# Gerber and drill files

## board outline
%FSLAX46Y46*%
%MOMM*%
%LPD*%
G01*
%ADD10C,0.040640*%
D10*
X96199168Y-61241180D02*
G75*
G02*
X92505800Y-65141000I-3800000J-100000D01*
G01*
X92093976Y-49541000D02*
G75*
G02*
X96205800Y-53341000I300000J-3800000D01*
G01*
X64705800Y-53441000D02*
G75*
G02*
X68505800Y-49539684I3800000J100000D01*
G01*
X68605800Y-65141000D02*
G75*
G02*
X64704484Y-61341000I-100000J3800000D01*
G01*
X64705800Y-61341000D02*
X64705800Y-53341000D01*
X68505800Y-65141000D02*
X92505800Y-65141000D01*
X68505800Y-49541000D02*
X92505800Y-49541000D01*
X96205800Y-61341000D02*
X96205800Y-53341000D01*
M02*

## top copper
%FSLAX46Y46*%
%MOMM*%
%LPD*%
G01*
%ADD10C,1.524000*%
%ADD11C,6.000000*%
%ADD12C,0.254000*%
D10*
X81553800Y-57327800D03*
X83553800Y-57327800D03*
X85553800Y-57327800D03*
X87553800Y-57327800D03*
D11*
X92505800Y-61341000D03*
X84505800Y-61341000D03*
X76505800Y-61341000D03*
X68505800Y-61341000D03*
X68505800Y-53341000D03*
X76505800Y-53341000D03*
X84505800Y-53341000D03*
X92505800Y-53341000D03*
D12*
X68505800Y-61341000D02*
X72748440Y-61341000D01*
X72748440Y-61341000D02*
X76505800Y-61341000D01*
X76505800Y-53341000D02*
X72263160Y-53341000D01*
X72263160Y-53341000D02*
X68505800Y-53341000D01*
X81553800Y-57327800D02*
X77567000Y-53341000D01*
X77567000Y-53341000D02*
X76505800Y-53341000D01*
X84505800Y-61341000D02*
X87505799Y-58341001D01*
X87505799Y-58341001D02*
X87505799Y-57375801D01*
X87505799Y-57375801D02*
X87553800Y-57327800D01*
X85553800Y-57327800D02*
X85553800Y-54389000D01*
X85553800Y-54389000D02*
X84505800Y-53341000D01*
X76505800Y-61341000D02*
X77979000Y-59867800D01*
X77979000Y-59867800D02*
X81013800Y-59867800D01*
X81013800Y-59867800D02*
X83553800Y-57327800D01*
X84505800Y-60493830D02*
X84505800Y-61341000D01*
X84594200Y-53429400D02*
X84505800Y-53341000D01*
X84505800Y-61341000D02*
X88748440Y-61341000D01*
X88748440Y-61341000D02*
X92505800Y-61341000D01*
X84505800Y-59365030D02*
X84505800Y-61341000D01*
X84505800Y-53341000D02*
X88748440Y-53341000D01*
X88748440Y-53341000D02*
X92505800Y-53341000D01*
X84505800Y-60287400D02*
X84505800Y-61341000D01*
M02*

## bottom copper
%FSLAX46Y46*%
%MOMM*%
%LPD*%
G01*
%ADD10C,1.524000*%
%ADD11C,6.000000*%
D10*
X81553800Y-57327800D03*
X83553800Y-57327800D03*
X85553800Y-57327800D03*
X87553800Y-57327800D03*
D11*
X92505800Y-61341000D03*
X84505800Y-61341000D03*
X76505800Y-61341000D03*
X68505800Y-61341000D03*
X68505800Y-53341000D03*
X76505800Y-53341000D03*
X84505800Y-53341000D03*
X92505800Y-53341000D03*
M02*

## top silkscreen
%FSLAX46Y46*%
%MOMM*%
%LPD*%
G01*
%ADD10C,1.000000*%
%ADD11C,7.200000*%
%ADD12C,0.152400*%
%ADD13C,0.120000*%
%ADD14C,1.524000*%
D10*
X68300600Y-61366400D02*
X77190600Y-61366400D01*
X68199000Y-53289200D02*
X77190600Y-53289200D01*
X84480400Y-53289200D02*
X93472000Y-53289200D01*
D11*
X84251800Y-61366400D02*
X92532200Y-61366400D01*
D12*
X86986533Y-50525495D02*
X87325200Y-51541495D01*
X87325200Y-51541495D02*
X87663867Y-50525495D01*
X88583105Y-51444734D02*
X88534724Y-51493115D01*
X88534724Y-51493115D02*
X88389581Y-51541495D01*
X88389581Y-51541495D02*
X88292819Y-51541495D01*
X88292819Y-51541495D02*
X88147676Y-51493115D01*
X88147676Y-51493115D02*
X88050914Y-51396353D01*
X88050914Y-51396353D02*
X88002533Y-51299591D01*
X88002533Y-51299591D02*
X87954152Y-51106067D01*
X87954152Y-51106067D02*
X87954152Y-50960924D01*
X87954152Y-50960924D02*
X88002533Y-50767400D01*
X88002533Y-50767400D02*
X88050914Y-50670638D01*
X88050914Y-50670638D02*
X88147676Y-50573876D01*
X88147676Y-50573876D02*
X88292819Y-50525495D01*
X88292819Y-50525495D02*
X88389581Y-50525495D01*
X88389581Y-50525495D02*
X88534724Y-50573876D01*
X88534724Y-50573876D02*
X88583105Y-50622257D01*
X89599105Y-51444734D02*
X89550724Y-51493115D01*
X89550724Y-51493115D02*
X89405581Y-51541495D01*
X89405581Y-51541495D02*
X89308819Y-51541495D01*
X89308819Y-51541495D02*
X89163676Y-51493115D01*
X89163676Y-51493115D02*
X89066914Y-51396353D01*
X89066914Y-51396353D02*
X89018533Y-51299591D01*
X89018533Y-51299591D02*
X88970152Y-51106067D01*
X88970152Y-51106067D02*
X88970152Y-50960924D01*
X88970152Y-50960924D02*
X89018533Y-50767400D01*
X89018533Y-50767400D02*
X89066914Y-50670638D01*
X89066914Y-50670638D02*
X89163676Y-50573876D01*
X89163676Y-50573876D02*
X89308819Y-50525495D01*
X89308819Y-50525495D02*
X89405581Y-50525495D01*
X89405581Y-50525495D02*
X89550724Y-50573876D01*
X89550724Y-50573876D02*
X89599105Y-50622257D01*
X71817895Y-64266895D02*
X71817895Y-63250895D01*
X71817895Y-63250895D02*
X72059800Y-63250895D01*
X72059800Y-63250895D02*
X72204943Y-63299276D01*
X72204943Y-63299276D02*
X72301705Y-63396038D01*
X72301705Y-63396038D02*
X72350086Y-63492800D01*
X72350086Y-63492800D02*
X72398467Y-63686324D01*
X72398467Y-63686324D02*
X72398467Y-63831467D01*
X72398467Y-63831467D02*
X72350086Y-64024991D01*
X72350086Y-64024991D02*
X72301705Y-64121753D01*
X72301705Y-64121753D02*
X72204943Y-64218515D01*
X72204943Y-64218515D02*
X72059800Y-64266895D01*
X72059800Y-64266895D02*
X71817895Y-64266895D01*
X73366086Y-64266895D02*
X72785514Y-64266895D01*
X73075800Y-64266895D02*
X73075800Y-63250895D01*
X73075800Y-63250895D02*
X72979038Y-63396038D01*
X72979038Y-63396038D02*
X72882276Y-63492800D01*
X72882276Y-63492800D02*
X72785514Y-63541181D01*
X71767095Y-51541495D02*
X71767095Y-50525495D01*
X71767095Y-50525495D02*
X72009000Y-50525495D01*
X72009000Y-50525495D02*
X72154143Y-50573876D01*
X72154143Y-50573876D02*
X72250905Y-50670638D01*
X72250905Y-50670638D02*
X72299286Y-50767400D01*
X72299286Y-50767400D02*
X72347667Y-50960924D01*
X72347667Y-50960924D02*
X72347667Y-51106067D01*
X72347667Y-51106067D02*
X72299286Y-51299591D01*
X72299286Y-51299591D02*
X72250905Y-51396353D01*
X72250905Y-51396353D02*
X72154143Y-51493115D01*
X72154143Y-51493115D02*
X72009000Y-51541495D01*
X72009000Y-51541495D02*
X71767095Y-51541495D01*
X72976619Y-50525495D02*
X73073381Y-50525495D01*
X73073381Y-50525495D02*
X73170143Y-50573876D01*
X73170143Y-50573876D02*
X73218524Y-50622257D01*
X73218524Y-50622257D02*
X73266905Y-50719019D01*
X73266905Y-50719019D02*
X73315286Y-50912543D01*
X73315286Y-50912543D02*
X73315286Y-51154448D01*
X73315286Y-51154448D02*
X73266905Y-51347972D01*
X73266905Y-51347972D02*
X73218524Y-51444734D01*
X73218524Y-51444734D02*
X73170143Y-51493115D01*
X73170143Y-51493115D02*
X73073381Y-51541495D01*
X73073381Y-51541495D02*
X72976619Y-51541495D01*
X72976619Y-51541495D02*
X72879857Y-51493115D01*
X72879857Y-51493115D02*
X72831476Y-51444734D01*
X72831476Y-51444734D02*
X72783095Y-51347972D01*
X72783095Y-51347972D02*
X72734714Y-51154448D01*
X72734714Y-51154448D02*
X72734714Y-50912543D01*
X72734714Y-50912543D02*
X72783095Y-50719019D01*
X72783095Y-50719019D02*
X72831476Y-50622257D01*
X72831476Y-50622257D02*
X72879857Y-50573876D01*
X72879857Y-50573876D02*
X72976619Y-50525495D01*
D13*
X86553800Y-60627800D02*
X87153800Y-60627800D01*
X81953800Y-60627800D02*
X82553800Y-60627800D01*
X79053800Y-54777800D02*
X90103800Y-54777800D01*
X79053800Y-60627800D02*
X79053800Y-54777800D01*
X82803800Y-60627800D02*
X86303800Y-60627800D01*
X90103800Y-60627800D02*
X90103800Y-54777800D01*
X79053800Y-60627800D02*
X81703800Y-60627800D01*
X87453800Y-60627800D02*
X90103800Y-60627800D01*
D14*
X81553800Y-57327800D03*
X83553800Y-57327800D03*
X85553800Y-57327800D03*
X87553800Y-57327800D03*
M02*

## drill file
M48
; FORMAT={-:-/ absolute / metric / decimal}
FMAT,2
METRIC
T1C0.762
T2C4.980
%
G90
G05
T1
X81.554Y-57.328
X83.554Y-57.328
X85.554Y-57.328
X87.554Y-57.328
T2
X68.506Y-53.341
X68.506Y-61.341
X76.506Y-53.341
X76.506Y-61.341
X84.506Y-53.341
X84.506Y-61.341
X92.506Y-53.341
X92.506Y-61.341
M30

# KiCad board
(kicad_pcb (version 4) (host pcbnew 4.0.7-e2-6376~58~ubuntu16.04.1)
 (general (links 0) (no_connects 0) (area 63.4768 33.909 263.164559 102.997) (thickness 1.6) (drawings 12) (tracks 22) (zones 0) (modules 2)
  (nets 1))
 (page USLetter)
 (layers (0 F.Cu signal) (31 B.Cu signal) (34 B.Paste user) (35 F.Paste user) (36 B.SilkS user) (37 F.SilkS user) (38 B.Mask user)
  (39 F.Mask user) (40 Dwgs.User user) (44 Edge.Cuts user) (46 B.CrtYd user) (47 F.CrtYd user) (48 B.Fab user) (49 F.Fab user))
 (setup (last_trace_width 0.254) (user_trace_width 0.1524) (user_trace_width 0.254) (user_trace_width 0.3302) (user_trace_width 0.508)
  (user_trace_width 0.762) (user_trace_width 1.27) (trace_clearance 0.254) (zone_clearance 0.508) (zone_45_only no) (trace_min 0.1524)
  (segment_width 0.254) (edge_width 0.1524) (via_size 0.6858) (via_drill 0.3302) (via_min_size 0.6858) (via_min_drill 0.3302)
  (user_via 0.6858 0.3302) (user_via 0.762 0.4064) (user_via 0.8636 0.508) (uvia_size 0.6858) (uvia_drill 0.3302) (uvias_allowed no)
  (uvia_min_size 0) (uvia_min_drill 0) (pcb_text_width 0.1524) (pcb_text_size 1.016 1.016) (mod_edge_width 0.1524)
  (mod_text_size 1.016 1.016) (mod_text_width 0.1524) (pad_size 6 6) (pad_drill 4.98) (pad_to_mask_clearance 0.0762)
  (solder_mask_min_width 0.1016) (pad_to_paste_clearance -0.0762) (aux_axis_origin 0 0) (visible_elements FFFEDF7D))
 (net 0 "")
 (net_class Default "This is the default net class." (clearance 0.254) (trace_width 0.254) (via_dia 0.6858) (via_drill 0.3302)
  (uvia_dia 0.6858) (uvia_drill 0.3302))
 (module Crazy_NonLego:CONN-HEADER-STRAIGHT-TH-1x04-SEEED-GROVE (layer F.Cu) (at 81.5538 57.3278 90)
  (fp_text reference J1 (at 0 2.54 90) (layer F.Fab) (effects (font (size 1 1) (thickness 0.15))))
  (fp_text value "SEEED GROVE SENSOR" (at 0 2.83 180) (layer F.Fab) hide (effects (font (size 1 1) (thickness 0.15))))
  (fp_line (start -3.3 5) (end -3.3 5.6) (layer F.SilkS) (width 0.12))
  (fp_line (start -3.3 0.4) (end -3.3 1) (layer F.SilkS) (width 0.12))
  (fp_line (start 2.55 -2.5) (end 2.55 8.55) (layer F.SilkS) (width 0.12))
  (fp_line (start -3.3 -2.5) (end 2.55 -2.5) (layer F.SilkS) (width 0.12))
  (fp_line (start -3.3 1.25) (end -3.3 4.75) (layer F.SilkS) (width 0.12))
  (fp_line (start -3.3 8.55) (end 2.55 8.55) (layer F.SilkS) (width 0.12))
  (fp_line (start -3.3 -2.5) (end -3.3 0.15) (layer F.SilkS) (width 0.12))
  (fp_line (start -3.3 5.9) (end -3.3 8.55) (layer F.SilkS) (width 0.12))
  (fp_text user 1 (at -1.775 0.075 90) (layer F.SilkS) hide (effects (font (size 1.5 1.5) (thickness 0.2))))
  (pad 1 thru_hole circle (at 0 0 90) (size 1.524 1.524) (drill 0.762) (layers *.Cu *.Mask F.SilkS))
  (pad 2 thru_hole circle (at 0 2 90) (size 1.524 1.524) (drill 0.762) (layers *.Cu *.Mask F.SilkS))
  (pad 3 thru_hole circle (at 0 4 90) (size 1.524 1.524) (drill 0.762) (layers *.Cu *.Mask F.SilkS))
  (pad 4 thru_hole circle (at 0 6 90) (size 1.524 1.524) (drill 0.762) (layers *.Cu *.Mask F.SilkS)))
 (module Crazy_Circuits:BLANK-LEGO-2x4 (layer F.Cu) (at 92.5058 61.341 90)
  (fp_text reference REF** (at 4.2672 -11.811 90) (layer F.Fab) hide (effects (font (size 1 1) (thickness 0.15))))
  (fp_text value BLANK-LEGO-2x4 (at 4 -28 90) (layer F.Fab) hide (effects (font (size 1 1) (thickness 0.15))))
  (fp_arc (start -0.00018 -0.106632) (end 0.09982 3.693368) (angle 89.9) (layer Edge.Cuts) (width 0.04064))
  (fp_arc (start 8 -0.111824) (end 11.8 -0.411824) (angle 94.51398846) (layer Edge.Cuts) (width 0.04064))
  (fp_arc (start 8 -24) (end 7.9 -27.8) (angle 91.50743576) (layer Edge.Cuts) (width 0.04064))
  (fp_arc (start 0 -24) (end -3.8 -23.9) (angle 91.50743576) (layer Edge.Cuts) (width 0.04064))
  (fp_line (start 0 -27.8) (end 8 -27.8) (layer Edge.Cuts) (width 0.04064))
  (fp_line (start -3.8 -24) (end -3.8 0) (layer Edge.Cuts) (width 0.04064))
  (fp_line (start 11.8 -24) (end 11.8 0) (layer Edge.Cuts) (width 0.04064))
  (fp_line (start 0 3.7) (end 8 3.7) (layer Edge.Cuts) (width 0.04064))
  (pad 4 thru_hole circle (at 0 0 90) (size 6 6) (drill 4.98) (layers *.Cu *.Mask))
  (pad 4 thru_hole circle (at 0 -8 90) (size 6 6) (drill 4.98) (layers *.Cu))
  (pad 2 thru_hole circle (at 0 -16 90) (size 6 6) (drill 4.98) (layers *.Cu *.Mask))
  (pad 2 thru_hole circle (at 0 -24 90) (size 6 6) (drill 4.98) (layers *.Cu *.Mask))
  (pad 1 thru_hole circle (at 8 -24 90) (size 6 6) (drill 4.98) (layers *.Cu *.Mask))
  (pad 1 thru_hole circle (at 8 -16 90) (size 6 6) (drill 4.98) (layers *.Cu *.Mask))
  (pad 3 thru_hole circle (at 8 -8 90) (size 6 6) (drill 4.98) (layers *.Cu))
  (pad 3 thru_hole circle (at 8 0 90) (size 6 6) (drill 4.98) (layers *.Cu *.Mask)))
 (gr_line (start 68.3006 61.3664) (end 77.1906 61.3664) (layer F.SilkS) (width 1))
 (gr_line (start 68.199 53.2892) (end 77.1906 53.2892) (layer F.SilkS) (width 1))
 (gr_line (start 84.4804 53.2892) (end 93.472 53.2892) (layer F.SilkS) (width 1))
 (gr_line (start 84.2518 61.3664) (end 92.5322 61.3664) (layer F.SilkS) (width 7.2))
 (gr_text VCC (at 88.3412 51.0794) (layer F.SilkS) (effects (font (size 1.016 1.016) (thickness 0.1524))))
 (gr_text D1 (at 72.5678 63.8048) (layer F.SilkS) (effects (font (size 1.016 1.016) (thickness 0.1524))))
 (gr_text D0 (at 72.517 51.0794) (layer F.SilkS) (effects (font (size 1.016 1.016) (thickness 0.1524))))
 (segment (start 68.5058 61.341) (end 72.74844 61.341) (width 0.254) (layer F.Cu) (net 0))
 (segment (start 72.74844 61.341) (end 76.5058 61.341) (width 0.254) (layer F.Cu) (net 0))
 (segment (start 76.5058 53.341) (end 72.26316 53.341) (width 0.254) (layer F.Cu) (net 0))
 (segment (start 72.26316 53.341) (end 68.5058 53.341) (width 0.254) (layer F.Cu) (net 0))
 (segment (start 81.5538 57.3278) (end 77.567 53.341) (width 0.254) (layer F.Cu) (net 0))
 (segment (start 77.567 53.341) (end 76.5058 53.341) (width 0.254) (layer F.Cu) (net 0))
 (segment (start 84.5058 61.341) (end 87.505799 58.341001) (width 0.254) (layer F.Cu) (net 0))
 (segment (start 87.505799 58.341001) (end 87.505799 57.375801) (width 0.254) (layer F.Cu) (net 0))
 (segment (start 87.505799 57.375801) (end 87.5538 57.3278) (width 0.254) (layer F.Cu) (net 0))
 (segment (start 85.5538 57.3278) (end 85.5538 54.389) (width 0.254) (layer F.Cu) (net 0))
 (segment (start 85.5538 54.389) (end 84.5058 53.341) (width 0.254) (layer F.Cu) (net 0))
 (segment (start 76.5058 61.341) (end 77.979 59.8678) (width 0.254) (layer F.Cu) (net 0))
 (segment (start 77.979 59.8678) (end 81.0138 59.8678) (width 0.254) (layer F.Cu) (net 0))
 (segment (start 81.0138 59.8678) (end 83.5538 57.3278) (width 0.254) (layer F.Cu) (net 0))
 (segment (start 84.5058 60.49383) (end 84.5058 61.341) (width 0.254) (layer F.Cu) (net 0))
 (segment (start 84.5942 53.4294) (end 84.5058 53.341) (width 0.254) (layer F.Cu) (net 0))
 (segment (start 84.5058 61.341) (end 88.74844 61.341) (width 0.254) (layer F.Cu) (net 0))
 (segment (start 88.74844 61.341) (end 92.5058 61.341) (width 0.254) (layer F.Cu) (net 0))
 (segment (start 84.5058 59.36503) (end 84.5058 61.341) (width 0.254) (layer F.Cu) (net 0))
 (segment (start 84.5058 53.341) (end 88.74844 53.341) (width 0.254) (layer F.Cu) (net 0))
 (segment (start 88.74844 53.341) (end 92.5058 53.341) (width 0.254) (layer F.Cu) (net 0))
 (segment (start 84.5058 60.2874) (end 84.5058 61.341) (width 0.254) (layer F.Cu) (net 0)))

